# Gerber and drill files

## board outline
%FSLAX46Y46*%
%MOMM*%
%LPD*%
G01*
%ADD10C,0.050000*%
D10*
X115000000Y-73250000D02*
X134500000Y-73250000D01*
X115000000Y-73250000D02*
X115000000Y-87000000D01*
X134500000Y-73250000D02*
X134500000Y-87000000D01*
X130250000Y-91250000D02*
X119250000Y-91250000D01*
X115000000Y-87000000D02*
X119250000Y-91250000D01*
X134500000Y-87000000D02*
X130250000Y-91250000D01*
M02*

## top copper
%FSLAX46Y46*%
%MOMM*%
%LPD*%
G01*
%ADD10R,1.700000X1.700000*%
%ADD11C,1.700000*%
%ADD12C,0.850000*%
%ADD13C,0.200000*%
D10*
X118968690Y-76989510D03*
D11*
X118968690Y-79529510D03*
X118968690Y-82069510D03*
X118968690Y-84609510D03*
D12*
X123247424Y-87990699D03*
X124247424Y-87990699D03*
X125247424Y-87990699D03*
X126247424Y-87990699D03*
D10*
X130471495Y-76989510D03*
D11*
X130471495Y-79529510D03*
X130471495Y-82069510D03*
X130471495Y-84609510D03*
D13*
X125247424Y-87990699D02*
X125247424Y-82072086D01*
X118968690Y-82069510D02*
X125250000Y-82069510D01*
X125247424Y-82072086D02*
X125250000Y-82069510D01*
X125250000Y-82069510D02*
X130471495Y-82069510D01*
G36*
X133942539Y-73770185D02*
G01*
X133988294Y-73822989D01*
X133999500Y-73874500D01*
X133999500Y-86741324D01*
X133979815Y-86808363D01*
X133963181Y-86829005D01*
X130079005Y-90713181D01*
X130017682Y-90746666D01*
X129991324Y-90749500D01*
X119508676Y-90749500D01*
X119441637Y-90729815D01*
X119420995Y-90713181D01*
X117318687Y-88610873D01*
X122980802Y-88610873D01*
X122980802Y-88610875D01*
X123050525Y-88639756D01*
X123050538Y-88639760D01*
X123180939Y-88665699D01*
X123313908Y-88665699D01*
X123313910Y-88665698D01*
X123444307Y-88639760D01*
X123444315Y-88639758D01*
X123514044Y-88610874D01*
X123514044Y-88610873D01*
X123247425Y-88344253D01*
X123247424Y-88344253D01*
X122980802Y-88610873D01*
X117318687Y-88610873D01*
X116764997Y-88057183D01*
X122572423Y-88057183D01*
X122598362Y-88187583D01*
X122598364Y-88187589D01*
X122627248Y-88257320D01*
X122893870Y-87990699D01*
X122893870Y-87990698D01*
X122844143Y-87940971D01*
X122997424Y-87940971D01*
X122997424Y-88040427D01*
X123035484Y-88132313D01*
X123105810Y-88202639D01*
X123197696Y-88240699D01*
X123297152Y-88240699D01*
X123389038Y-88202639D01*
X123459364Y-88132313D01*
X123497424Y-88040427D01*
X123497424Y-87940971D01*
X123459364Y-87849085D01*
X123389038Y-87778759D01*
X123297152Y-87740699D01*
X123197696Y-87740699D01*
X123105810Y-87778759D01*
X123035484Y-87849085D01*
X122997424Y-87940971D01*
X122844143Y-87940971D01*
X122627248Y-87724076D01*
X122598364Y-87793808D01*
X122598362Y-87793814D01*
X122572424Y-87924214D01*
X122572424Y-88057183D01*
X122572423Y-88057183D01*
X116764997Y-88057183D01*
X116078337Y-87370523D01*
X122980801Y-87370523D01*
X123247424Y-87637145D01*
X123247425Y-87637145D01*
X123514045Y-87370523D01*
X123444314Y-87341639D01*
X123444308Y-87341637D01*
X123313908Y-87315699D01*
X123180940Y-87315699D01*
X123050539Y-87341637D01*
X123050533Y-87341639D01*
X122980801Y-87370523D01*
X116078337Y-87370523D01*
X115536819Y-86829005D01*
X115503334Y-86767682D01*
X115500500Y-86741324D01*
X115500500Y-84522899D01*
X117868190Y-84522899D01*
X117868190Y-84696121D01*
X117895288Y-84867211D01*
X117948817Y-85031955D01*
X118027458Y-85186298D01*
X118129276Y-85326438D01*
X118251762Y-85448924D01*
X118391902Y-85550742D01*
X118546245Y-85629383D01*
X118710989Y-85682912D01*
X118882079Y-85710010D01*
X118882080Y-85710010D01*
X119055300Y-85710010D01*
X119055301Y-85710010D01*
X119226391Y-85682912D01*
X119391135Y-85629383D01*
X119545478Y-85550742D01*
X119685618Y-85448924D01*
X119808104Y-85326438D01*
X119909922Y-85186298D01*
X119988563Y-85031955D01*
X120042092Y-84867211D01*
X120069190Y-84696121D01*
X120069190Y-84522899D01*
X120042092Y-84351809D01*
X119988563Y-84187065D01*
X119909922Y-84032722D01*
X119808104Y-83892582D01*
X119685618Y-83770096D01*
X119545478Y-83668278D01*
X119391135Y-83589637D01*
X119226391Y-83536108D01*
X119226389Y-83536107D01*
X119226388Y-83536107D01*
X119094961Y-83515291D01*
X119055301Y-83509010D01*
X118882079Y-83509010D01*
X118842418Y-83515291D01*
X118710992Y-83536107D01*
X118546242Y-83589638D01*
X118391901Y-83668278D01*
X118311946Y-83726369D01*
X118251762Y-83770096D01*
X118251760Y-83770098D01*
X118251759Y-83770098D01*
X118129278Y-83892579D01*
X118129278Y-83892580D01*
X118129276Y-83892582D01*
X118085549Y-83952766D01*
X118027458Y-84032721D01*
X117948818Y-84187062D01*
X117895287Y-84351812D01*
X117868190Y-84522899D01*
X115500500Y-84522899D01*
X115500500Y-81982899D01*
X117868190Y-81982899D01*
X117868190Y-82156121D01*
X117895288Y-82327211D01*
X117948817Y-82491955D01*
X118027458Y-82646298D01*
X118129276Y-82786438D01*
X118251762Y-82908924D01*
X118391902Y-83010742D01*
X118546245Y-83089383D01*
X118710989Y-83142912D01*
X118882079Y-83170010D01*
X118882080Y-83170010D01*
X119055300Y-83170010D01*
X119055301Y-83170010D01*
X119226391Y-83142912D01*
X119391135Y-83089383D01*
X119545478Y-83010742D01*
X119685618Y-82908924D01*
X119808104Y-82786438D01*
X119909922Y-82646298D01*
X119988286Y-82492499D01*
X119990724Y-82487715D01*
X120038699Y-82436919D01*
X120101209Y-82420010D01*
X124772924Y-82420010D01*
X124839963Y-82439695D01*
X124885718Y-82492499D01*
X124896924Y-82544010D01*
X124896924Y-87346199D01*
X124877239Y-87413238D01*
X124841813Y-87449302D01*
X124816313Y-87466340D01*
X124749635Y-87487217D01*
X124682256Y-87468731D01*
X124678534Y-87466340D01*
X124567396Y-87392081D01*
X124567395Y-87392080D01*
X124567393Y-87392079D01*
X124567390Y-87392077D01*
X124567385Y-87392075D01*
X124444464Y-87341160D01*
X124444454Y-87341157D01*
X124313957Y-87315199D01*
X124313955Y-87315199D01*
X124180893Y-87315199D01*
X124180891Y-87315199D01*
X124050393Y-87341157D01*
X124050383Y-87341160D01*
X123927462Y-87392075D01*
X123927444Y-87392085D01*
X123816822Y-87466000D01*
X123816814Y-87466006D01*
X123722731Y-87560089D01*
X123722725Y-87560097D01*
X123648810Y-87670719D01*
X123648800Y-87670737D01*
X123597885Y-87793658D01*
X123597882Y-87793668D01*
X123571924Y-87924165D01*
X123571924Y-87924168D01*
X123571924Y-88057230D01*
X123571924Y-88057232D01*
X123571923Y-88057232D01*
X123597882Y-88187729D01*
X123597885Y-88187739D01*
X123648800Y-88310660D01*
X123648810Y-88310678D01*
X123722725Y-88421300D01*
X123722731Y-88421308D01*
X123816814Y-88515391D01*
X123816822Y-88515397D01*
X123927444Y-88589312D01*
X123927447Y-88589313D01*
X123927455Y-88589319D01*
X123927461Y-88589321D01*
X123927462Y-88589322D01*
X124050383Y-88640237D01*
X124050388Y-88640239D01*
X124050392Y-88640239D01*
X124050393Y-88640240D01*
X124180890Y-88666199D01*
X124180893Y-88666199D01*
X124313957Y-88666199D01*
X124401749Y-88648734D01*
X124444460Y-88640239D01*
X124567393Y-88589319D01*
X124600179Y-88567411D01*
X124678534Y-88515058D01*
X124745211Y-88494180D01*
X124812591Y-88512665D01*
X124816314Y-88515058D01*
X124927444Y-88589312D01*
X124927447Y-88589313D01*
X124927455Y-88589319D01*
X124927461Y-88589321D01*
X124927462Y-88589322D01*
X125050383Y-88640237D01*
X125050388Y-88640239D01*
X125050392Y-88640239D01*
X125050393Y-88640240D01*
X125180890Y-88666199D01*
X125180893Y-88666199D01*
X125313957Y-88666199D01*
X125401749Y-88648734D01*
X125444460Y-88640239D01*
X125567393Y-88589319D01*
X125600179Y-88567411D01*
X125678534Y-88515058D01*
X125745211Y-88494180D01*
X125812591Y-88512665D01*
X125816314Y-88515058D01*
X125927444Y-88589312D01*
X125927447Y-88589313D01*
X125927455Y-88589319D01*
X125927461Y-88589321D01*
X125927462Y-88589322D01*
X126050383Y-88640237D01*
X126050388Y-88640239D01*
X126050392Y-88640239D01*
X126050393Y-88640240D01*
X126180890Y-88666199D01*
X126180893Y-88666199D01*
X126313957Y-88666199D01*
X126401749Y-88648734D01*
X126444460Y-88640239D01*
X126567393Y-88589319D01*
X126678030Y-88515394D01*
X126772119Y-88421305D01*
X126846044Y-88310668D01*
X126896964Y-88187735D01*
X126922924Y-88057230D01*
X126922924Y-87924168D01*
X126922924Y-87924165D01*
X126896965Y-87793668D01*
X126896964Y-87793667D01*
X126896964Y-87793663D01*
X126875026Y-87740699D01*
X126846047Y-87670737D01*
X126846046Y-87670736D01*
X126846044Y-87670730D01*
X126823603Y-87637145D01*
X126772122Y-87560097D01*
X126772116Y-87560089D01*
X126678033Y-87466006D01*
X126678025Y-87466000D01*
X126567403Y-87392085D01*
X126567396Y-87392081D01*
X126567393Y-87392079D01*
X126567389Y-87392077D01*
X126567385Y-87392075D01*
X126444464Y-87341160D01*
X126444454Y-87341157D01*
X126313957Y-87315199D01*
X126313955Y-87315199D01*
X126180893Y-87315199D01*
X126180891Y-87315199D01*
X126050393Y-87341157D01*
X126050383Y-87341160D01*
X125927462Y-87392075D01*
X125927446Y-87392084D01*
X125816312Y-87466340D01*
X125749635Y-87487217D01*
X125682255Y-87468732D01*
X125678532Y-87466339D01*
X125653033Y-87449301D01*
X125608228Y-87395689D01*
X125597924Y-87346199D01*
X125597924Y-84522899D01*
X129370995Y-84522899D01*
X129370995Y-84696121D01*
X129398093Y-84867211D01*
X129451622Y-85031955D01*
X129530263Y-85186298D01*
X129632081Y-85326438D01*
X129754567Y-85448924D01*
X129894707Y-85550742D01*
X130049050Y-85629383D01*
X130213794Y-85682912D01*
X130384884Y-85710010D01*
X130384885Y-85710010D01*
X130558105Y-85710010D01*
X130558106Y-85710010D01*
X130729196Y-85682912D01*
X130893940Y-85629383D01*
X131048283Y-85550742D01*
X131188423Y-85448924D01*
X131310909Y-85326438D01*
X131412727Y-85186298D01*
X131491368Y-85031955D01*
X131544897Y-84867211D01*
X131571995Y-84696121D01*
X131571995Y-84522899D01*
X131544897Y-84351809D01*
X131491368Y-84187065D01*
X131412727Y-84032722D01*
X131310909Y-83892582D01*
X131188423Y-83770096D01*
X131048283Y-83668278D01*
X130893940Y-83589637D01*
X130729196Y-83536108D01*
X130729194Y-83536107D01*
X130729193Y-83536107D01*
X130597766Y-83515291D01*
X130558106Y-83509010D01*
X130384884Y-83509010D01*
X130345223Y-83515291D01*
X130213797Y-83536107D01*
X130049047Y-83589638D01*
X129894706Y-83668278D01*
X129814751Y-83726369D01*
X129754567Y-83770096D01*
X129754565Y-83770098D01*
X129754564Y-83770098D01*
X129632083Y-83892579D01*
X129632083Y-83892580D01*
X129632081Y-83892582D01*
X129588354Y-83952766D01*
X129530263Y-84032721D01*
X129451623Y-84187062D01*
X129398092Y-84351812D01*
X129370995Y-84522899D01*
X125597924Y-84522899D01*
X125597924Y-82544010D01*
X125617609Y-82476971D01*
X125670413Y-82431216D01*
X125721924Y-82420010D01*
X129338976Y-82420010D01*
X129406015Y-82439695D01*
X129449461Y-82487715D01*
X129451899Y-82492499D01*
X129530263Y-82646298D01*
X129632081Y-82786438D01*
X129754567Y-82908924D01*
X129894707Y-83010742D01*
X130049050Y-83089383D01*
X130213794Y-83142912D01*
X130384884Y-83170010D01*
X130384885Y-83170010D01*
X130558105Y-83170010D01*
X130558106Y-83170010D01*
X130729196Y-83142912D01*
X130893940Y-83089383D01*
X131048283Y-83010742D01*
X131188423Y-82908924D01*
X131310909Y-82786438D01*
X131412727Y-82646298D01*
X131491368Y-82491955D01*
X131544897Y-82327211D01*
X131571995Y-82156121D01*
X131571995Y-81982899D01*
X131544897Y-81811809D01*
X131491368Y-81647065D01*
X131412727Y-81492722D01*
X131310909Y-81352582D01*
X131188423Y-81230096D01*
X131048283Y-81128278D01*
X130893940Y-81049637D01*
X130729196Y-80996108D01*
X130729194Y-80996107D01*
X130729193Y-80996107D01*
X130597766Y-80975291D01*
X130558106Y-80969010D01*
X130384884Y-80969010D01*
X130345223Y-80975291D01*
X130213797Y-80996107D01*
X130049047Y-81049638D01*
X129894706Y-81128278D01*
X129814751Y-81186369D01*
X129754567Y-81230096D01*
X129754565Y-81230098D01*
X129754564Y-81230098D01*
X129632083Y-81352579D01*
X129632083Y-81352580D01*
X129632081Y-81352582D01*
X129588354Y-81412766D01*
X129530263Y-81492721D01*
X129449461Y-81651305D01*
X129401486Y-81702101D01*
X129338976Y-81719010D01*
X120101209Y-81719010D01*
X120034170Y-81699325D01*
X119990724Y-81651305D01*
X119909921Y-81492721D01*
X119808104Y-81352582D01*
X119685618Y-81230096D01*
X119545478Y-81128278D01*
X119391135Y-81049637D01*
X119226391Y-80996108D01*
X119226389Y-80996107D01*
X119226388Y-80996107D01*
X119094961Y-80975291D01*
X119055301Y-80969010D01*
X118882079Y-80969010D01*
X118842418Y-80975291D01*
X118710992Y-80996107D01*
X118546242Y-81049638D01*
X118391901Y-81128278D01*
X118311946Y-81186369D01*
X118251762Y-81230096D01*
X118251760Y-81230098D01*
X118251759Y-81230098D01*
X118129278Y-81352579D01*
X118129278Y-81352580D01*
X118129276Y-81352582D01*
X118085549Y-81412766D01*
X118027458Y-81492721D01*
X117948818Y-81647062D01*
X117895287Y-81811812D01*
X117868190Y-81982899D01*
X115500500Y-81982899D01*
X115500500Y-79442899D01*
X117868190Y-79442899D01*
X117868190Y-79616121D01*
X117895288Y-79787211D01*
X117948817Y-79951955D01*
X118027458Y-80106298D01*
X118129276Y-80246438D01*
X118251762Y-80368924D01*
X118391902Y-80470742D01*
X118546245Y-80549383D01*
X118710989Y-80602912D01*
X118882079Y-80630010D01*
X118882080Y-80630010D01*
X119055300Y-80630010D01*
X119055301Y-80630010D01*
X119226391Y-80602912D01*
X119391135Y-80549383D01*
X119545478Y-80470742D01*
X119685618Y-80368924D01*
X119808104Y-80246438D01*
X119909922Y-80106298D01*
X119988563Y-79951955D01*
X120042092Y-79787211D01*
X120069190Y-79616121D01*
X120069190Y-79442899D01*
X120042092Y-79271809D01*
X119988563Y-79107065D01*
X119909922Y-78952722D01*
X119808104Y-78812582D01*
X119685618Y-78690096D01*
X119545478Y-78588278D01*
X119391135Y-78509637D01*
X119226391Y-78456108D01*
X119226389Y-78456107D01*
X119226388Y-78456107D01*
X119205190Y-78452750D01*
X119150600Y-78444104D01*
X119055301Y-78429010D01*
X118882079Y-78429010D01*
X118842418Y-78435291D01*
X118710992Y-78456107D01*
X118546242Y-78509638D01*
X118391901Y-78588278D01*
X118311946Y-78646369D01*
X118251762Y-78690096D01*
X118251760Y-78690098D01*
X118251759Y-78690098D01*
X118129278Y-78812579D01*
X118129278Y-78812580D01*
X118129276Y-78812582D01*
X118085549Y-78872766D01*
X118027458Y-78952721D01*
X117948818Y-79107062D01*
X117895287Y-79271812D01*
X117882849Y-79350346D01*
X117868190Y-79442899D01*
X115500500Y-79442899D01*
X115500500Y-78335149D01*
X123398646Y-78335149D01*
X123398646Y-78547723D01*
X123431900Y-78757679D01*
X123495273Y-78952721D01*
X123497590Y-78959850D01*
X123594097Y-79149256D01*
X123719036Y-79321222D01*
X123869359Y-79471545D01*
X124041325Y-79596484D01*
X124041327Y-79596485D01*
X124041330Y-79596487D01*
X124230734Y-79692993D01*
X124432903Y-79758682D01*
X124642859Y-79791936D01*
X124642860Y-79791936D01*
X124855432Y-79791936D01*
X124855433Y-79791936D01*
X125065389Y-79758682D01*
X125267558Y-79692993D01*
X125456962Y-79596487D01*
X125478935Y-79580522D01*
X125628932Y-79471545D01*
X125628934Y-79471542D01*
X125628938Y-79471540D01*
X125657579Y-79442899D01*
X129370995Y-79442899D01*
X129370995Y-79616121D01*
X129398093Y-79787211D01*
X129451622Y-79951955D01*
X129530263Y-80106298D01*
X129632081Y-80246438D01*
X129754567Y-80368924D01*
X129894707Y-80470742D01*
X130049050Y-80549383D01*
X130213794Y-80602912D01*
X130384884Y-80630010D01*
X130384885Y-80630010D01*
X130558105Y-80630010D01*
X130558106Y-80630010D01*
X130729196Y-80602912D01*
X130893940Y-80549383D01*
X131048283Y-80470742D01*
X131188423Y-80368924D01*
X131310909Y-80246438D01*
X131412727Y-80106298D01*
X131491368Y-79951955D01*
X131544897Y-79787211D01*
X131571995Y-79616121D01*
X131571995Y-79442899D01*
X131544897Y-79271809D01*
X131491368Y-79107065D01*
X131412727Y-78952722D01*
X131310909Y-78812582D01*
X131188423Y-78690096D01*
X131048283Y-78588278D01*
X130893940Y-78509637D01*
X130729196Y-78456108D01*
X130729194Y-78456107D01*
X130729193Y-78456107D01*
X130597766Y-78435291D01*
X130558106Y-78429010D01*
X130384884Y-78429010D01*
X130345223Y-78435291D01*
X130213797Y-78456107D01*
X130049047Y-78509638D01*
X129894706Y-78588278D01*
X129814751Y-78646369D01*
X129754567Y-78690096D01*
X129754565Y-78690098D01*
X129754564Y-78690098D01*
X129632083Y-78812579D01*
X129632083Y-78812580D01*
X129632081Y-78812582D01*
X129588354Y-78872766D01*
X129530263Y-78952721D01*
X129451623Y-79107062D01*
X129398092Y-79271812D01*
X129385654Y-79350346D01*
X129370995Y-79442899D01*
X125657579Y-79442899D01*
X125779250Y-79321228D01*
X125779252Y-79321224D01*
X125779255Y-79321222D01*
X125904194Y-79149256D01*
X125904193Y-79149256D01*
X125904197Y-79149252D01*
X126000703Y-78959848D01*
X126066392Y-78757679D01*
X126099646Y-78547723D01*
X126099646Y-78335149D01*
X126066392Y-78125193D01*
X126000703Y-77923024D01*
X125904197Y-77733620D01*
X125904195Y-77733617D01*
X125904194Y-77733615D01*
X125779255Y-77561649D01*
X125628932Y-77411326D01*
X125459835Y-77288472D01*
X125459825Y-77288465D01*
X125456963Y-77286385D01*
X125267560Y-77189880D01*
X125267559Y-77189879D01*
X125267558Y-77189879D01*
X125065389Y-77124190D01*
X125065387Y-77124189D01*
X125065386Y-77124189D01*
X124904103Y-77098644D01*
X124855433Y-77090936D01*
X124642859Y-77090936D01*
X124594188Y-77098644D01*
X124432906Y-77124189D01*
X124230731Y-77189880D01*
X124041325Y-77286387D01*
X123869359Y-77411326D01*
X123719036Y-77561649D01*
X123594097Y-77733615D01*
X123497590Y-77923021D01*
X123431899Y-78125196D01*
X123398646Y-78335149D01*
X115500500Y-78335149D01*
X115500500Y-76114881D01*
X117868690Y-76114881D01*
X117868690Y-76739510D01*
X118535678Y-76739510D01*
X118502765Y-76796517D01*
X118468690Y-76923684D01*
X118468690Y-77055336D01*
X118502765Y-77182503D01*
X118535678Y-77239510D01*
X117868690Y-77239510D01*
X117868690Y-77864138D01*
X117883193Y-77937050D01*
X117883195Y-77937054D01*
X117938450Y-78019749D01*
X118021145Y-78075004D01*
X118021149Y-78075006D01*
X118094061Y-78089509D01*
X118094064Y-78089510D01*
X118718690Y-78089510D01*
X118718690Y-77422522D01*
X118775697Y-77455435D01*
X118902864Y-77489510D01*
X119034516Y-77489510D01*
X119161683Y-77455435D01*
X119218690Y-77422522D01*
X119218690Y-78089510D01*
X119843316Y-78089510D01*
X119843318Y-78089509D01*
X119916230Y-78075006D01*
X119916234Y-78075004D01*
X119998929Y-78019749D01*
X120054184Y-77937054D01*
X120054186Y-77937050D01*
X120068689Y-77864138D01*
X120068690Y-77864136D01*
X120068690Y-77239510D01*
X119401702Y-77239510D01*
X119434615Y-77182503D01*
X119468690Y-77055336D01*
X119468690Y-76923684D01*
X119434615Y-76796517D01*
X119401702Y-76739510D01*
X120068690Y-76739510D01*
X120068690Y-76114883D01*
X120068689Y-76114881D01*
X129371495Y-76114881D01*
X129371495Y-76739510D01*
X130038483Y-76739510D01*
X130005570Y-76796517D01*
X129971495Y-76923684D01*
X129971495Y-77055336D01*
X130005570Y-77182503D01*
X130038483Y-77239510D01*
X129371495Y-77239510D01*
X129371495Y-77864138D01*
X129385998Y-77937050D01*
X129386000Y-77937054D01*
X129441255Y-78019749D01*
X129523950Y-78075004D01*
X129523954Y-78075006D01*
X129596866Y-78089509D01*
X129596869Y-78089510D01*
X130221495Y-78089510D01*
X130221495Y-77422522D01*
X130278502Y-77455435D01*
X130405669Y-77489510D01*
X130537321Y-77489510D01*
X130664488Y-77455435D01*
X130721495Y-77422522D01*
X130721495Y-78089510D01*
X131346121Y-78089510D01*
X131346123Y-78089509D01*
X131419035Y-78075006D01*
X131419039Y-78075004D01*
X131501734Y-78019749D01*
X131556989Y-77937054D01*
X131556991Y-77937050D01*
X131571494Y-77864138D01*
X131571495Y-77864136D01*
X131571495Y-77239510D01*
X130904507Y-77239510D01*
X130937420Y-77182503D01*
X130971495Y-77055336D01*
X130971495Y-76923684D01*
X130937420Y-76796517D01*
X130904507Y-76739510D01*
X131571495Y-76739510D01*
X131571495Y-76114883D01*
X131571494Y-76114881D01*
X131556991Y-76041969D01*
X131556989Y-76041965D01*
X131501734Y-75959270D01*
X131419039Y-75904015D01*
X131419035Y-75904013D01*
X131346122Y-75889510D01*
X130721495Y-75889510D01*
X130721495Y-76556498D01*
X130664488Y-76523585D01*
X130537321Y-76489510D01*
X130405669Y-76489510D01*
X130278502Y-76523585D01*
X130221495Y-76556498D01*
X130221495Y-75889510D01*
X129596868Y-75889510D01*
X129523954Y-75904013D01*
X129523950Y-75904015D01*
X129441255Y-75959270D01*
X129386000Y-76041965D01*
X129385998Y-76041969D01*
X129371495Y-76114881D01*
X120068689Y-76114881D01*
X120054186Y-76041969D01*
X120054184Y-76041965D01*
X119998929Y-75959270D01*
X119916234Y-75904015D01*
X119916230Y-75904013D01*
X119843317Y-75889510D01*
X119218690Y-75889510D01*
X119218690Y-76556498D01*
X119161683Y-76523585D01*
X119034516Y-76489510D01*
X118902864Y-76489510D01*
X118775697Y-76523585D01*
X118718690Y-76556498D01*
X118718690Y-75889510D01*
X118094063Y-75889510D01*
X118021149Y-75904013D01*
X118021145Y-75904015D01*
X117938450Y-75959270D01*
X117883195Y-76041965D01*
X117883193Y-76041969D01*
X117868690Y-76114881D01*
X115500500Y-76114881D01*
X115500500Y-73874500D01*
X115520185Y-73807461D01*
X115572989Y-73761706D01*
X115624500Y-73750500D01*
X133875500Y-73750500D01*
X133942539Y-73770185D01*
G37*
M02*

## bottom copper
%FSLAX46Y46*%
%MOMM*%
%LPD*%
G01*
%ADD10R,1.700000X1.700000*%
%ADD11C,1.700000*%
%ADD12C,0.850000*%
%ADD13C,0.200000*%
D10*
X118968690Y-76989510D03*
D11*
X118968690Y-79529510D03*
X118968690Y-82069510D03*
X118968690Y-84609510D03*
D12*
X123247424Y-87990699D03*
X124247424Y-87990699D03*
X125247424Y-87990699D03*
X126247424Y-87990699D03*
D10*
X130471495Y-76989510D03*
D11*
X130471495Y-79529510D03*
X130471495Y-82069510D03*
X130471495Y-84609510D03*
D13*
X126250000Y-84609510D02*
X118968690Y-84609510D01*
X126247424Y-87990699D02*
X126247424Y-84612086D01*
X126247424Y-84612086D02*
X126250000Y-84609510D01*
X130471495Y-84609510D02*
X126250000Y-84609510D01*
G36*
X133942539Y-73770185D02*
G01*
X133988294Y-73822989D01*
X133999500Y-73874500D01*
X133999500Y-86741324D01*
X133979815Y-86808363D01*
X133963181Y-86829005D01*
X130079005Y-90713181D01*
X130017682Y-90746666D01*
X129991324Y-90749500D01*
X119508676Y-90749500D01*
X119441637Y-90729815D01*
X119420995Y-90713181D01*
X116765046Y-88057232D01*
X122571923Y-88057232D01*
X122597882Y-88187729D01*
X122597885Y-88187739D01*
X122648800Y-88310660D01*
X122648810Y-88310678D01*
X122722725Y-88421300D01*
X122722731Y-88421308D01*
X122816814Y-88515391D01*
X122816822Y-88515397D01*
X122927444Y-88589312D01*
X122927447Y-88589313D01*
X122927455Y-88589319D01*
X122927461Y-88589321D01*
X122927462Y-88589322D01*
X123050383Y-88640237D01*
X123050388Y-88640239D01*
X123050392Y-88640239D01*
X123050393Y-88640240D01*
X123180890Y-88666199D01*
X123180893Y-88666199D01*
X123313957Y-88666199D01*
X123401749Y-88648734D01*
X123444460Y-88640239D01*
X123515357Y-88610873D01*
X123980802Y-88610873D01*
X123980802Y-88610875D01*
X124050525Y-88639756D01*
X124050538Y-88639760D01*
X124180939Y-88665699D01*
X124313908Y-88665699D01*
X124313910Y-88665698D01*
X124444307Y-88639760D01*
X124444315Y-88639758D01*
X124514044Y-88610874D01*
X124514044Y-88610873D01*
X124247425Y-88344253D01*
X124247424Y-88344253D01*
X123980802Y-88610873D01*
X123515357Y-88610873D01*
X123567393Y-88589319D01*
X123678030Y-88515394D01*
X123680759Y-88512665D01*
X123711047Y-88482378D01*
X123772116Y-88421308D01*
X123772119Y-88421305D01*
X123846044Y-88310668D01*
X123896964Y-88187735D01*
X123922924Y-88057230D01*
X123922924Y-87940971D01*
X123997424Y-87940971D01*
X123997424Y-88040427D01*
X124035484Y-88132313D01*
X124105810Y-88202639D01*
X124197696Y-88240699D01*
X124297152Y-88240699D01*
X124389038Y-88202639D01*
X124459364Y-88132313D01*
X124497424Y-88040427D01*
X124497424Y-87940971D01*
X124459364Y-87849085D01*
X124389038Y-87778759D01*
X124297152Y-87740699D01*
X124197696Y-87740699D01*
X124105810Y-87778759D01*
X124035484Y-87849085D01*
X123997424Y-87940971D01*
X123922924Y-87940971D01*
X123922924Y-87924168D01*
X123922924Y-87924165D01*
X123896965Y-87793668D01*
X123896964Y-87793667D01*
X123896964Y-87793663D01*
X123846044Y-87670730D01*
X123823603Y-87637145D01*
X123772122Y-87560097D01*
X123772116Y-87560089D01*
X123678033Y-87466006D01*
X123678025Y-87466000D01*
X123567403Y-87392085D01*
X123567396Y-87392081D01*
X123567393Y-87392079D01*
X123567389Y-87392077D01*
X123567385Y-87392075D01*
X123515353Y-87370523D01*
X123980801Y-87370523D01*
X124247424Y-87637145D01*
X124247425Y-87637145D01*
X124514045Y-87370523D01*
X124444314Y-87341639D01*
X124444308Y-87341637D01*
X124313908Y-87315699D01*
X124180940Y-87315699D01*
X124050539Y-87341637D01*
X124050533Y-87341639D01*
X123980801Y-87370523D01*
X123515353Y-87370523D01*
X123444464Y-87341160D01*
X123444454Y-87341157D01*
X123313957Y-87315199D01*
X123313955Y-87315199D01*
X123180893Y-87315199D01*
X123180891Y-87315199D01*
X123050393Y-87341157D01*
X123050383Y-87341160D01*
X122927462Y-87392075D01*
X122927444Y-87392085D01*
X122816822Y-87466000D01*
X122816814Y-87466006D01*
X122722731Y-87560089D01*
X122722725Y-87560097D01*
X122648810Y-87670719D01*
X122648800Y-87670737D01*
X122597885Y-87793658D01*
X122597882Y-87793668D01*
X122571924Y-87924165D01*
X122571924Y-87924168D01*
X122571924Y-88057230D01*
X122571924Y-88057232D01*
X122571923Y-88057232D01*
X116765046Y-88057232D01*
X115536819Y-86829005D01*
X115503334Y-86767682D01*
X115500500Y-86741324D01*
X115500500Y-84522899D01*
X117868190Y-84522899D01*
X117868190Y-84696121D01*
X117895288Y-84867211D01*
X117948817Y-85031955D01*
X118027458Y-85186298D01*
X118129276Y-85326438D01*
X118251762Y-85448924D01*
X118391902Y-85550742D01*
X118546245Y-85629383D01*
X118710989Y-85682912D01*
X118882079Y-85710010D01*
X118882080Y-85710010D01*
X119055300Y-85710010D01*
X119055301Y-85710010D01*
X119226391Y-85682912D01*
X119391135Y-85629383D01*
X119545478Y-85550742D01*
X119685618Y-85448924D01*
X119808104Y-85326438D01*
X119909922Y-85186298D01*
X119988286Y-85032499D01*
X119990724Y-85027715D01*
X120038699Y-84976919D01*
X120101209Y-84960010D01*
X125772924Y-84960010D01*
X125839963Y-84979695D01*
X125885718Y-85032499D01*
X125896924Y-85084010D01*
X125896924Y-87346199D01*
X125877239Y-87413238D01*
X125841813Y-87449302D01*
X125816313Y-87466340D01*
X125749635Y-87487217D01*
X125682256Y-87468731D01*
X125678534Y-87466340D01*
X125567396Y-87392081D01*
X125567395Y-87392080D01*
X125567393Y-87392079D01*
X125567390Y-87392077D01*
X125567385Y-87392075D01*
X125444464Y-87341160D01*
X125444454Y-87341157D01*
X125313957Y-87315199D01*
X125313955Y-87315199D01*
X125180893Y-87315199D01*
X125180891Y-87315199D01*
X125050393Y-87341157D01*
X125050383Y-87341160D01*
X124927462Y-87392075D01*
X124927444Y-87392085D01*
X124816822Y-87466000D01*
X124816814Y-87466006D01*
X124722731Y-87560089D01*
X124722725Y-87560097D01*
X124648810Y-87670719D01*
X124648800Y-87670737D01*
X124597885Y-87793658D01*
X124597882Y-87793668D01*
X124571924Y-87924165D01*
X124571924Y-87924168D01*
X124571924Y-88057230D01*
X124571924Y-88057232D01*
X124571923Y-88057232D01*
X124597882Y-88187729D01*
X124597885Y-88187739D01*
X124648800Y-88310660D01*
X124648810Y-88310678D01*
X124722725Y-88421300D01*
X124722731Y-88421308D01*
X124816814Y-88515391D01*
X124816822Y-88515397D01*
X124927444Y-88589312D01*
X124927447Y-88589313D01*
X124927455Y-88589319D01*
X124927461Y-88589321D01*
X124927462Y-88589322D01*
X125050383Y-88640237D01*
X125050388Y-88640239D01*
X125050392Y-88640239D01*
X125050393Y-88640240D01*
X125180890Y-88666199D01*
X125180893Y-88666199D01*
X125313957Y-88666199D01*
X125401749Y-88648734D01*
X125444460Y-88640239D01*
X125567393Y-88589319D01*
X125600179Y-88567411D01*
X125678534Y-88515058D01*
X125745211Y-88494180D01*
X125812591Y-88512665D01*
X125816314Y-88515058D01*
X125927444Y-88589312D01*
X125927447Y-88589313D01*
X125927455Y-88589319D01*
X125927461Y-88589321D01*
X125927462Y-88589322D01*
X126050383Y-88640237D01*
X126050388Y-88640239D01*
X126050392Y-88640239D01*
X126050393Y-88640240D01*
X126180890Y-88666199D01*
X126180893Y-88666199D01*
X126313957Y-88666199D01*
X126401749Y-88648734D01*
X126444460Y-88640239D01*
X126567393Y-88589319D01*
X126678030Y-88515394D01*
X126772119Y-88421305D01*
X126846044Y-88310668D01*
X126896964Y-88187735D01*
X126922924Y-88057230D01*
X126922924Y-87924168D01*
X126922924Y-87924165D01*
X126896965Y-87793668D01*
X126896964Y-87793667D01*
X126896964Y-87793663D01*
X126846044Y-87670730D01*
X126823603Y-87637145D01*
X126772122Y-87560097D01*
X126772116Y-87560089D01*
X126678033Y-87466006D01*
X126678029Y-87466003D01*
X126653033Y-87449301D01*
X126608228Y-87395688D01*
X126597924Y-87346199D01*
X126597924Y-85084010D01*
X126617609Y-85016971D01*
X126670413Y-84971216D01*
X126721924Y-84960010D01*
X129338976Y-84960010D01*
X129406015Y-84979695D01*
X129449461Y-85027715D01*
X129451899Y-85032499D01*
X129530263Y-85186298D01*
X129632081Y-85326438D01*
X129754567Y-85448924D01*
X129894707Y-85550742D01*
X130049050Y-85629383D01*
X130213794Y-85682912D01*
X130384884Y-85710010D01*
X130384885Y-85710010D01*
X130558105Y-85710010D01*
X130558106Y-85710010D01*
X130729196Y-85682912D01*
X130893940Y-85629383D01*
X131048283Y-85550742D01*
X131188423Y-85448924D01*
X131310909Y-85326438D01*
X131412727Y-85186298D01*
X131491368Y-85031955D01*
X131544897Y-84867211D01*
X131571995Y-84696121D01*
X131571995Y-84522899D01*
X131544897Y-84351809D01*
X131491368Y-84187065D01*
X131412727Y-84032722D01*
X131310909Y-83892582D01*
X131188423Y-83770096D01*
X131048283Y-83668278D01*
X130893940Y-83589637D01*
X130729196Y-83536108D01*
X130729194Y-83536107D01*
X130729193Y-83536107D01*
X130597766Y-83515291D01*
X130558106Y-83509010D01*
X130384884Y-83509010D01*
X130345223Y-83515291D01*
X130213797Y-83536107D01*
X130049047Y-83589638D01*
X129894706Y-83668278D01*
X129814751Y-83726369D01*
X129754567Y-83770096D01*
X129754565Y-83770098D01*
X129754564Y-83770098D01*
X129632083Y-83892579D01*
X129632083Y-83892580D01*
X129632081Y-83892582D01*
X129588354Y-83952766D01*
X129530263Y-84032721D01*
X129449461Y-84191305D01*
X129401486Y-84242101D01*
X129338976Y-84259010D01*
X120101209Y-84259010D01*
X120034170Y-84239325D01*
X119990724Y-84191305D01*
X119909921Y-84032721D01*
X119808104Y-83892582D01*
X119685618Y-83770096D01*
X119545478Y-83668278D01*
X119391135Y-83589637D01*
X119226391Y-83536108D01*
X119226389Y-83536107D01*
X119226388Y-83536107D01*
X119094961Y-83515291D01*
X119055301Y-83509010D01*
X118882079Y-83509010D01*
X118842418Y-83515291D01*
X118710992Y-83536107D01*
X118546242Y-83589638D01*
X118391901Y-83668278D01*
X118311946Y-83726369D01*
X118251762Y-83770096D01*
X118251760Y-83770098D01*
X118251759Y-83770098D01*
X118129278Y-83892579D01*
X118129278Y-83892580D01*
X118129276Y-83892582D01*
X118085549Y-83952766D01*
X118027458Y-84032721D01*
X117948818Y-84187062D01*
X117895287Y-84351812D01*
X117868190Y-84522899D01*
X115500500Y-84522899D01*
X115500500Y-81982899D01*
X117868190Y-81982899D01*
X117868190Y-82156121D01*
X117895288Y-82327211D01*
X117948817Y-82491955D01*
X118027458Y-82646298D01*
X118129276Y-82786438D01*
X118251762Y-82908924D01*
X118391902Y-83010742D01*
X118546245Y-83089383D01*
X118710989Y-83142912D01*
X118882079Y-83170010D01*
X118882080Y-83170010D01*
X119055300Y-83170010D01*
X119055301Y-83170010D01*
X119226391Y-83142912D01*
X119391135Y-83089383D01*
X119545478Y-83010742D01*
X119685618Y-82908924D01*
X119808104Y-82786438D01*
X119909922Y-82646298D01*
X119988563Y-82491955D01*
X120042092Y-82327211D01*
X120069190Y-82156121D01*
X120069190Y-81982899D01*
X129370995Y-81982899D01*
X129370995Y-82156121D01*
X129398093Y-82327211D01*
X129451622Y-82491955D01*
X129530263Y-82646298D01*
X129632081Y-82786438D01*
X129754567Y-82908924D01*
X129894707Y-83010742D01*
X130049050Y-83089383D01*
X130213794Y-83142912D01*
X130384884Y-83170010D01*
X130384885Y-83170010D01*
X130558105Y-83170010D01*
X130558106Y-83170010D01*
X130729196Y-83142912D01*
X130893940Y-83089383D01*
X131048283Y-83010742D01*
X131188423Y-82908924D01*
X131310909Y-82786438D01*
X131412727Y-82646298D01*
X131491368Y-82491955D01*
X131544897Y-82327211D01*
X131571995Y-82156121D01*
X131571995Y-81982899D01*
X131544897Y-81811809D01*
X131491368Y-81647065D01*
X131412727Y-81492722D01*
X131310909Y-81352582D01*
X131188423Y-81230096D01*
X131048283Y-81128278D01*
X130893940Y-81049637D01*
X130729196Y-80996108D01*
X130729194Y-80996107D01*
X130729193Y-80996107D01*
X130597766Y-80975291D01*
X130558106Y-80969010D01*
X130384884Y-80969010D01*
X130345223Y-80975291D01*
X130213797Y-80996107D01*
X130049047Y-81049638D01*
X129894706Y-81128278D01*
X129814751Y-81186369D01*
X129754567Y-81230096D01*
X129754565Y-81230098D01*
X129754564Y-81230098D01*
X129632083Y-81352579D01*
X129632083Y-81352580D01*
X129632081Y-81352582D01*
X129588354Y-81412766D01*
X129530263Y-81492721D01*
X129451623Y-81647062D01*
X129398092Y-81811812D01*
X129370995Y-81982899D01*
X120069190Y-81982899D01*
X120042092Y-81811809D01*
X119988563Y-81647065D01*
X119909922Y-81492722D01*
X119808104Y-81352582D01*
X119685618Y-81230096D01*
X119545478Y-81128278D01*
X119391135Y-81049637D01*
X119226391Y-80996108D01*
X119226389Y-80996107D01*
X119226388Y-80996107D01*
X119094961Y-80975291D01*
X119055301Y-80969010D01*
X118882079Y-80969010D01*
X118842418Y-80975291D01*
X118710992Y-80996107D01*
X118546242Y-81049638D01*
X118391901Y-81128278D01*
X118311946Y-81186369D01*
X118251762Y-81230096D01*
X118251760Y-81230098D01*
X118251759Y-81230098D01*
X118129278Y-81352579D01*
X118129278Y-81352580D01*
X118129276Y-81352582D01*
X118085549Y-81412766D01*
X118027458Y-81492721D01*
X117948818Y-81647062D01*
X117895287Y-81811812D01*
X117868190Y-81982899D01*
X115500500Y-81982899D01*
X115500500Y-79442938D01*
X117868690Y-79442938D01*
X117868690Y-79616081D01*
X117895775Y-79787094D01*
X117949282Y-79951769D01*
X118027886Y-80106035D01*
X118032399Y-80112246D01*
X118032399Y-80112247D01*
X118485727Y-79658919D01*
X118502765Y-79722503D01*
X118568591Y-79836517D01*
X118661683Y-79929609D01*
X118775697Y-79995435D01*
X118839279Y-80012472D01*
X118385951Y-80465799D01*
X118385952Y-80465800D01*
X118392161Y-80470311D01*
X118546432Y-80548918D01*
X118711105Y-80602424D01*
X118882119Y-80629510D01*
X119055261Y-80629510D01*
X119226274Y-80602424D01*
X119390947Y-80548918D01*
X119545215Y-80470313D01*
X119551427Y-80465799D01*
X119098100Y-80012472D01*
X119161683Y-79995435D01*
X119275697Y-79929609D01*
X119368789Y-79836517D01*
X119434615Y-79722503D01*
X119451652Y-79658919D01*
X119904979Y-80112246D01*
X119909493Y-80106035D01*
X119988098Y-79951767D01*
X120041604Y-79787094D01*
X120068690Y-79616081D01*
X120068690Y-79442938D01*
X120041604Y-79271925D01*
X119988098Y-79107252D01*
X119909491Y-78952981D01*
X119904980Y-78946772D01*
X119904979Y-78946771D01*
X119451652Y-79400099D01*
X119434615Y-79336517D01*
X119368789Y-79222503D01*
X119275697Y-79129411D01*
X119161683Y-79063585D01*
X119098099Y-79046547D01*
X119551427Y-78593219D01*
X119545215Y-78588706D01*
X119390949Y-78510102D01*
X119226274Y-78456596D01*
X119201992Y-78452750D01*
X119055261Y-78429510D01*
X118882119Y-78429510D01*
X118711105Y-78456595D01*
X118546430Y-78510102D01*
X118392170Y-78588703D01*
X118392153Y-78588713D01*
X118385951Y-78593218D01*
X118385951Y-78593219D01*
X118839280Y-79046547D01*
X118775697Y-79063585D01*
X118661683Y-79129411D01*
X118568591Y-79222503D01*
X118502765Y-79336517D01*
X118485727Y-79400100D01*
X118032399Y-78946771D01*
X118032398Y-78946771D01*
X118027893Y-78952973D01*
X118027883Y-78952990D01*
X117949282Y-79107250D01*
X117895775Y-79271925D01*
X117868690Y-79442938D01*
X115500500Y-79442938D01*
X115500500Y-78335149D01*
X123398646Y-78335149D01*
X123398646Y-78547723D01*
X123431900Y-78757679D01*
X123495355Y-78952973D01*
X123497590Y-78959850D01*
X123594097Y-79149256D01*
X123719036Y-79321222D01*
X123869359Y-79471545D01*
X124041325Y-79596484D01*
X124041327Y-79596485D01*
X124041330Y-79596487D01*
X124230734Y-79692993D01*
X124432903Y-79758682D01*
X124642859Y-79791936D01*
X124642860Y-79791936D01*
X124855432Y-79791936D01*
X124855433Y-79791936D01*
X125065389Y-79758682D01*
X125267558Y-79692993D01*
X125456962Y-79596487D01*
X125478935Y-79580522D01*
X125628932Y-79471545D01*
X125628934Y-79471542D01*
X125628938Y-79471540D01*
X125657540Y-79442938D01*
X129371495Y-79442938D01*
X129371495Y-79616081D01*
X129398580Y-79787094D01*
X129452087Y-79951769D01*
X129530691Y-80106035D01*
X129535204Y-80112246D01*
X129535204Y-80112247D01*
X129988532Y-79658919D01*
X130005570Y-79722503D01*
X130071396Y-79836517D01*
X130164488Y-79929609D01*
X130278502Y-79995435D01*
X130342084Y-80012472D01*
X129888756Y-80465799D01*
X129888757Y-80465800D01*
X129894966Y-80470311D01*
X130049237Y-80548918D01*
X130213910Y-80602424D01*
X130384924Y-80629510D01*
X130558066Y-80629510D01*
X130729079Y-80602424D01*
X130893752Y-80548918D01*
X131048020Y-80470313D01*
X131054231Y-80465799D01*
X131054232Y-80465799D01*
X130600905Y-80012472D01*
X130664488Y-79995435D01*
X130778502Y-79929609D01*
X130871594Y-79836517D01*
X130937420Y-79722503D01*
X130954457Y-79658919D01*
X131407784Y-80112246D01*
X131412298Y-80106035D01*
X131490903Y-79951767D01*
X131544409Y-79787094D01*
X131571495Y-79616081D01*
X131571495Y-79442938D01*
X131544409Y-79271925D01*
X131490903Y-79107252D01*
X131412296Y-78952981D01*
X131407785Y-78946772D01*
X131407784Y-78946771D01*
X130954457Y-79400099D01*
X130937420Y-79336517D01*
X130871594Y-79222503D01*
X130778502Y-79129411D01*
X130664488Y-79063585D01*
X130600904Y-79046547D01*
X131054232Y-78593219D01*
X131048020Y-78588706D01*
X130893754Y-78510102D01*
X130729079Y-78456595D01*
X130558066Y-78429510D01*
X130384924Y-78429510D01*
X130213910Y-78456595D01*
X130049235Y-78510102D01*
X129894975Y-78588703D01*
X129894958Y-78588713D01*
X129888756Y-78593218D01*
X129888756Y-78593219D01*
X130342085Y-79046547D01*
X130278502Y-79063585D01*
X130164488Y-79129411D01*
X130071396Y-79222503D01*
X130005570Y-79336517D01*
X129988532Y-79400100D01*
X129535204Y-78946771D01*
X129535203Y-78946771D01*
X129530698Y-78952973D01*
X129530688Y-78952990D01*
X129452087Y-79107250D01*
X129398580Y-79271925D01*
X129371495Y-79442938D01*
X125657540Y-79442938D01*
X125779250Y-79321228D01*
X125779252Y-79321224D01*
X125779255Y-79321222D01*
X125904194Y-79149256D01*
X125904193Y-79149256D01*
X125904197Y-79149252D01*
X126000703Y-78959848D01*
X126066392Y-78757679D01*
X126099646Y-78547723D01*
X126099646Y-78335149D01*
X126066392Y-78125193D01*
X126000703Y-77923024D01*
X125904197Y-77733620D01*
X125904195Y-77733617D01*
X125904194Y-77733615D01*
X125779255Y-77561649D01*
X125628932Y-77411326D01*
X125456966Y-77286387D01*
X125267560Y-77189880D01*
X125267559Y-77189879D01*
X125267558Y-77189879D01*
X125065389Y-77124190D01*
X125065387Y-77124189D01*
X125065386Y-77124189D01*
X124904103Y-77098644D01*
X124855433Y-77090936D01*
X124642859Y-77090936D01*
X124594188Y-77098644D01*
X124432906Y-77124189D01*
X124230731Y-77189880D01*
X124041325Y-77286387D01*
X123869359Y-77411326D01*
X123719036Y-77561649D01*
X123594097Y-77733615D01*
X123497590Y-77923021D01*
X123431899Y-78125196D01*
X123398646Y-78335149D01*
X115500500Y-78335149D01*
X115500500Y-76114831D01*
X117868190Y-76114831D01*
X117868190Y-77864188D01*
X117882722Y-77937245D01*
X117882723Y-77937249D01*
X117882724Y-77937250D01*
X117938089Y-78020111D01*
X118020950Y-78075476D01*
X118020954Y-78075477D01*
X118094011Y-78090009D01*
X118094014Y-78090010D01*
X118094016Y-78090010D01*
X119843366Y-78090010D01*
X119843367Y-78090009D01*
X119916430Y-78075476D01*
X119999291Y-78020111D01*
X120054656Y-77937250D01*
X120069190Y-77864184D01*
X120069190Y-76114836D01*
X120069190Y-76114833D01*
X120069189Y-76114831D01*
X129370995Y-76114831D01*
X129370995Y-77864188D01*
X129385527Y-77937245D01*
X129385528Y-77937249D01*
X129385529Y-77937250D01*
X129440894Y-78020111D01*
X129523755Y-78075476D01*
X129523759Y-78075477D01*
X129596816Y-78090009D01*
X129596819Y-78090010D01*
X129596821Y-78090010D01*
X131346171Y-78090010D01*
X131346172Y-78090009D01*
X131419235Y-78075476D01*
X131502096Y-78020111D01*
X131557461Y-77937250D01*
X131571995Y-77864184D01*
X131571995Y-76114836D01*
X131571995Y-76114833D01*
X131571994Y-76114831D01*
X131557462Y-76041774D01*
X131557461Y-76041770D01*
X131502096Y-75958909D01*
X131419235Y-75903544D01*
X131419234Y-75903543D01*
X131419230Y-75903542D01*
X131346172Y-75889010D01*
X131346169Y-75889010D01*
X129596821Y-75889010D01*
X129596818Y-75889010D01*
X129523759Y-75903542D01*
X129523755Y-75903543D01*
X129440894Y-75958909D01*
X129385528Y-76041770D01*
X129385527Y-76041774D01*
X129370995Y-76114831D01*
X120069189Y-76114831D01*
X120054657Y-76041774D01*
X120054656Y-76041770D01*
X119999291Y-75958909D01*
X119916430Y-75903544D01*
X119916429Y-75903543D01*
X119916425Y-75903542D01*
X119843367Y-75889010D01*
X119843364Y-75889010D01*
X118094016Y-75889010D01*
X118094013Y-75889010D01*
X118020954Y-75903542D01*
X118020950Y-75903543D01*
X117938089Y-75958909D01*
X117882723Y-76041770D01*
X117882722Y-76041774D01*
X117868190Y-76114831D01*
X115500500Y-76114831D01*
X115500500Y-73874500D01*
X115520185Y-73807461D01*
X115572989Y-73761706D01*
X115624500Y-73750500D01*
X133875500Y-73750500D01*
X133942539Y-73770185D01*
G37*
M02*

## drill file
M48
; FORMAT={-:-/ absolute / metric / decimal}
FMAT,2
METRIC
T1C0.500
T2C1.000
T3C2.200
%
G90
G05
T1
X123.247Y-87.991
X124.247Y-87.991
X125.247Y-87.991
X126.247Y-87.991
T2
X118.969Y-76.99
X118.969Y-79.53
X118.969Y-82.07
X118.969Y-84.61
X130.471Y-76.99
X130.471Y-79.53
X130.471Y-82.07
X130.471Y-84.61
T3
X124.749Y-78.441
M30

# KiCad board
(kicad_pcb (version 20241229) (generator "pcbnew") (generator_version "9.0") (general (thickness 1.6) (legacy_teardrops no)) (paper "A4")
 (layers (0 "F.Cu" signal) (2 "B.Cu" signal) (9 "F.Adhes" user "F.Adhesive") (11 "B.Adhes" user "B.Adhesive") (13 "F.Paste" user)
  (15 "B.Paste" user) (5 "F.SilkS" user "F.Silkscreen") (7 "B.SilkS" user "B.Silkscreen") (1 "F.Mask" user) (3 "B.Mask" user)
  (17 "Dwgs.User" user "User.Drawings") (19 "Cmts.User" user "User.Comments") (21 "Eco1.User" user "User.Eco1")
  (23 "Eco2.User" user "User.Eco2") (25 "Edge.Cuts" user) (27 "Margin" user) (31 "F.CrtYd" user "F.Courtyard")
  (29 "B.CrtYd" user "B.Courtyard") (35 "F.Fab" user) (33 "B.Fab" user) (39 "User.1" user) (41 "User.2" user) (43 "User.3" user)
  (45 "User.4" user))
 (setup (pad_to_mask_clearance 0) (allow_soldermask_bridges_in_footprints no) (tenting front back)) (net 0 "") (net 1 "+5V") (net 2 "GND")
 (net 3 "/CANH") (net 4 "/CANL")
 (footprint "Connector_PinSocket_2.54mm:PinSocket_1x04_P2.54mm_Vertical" (layer "F.Cu") (at 118.96869 76.98951)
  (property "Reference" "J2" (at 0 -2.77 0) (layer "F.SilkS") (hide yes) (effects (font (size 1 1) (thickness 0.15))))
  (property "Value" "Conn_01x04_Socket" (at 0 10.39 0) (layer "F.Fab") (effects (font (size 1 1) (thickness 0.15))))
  (pad "1" thru_hole rect (at 0 0) (size 1.7 1.7) (drill 1) (layers "*.Cu" "*.Mask") (remove_unused_layers no) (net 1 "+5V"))
  (pad "2" thru_hole circle (at 0 2.54) (size 1.7 1.7) (drill 1) (layers "*.Cu" "*.Mask") (remove_unused_layers no) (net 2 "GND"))
  (pad "3" thru_hole circle (at 0 5.08) (size 1.7 1.7) (drill 1) (layers "*.Cu" "*.Mask") (remove_unused_layers no) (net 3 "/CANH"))
  (pad "4" thru_hole circle (at 0 7.62) (size 1.7 1.7) (drill 1) (layers "*.Cu" "*.Mask") (remove_unused_layers no) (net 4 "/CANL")))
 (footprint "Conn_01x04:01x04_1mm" (layer "F.Cu") (at 122.747424 88.490699 90)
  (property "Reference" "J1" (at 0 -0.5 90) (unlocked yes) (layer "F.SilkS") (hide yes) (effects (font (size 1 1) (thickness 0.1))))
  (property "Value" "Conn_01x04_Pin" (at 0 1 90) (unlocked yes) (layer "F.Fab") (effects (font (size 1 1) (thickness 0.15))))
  (pad "1" thru_hole circle (at 0.5 0.5 90) (size 0.85 0.85) (drill 0.5) (layers "*.Cu" "*.Mask") (remove_unused_layers no) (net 1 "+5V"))
  (pad "2" thru_hole circle (at 0.5 1.5 90) (size 0.85 0.85) (drill 0.5) (layers "*.Cu" "*.Mask") (remove_unused_layers no) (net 2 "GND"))
  (pad "3" thru_hole circle (at 0.5 2.5 90) (size 0.85 0.85) (drill 0.5) (layers "*.Cu" "*.Mask") (remove_unused_layers no) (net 3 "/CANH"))
  (pad "4" thru_hole circle (at 0.5 3.5 90) (size 0.85 0.85) (drill 0.5) (layers "*.Cu" "*.Mask") (remove_unused_layers no) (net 4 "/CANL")))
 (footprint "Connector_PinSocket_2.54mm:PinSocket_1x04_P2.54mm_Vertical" (layer "F.Cu") (at 130.471495 76.98951)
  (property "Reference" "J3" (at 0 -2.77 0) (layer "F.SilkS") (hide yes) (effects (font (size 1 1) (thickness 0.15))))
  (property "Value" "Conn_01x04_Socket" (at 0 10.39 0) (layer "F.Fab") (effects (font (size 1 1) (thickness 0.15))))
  (pad "1" thru_hole rect (at 0 0) (size 1.7 1.7) (drill 1) (layers "*.Cu" "*.Mask") (remove_unused_layers no) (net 1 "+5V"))
  (pad "2" thru_hole circle (at 0 2.54) (size 1.7 1.7) (drill 1) (layers "*.Cu" "*.Mask") (remove_unused_layers no) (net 2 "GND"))
  (pad "3" thru_hole circle (at 0 5.08) (size 1.7 1.7) (drill 1) (layers "*.Cu" "*.Mask") (remove_unused_layers no) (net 3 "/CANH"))
  (pad "4" thru_hole circle (at 0 7.62) (size 1.7 1.7) (drill 1) (layers "*.Cu" "*.Mask") (remove_unused_layers no) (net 4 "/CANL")))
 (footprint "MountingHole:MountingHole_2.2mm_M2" (layer "F.Cu") (at 124.749146 78.441436)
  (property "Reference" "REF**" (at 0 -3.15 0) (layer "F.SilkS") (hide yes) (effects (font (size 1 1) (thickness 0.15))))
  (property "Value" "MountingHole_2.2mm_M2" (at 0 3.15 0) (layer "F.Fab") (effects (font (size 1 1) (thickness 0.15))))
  (pad "" np_thru_hole circle (at 0 0) (size 2.2 2.2) (drill 2.2) (layers "*.Cu" "*.Mask")))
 (gr_line (start 115 73.25) (end 134.5 73.25) (stroke (width 0.05) (type solid)) (layer "Edge.Cuts"))
 (gr_line (start 115 73.25) (end 115 87) (stroke (width 0.05) (type default)) (layer "Edge.Cuts"))
 (gr_line (start 134.5 73.25) (end 134.5 87) (stroke (width 0.05) (type default)) (layer "Edge.Cuts"))
 (gr_line (start 130.25 91.25) (end 119.25 91.25) (stroke (width 0.05) (type default)) (layer "Edge.Cuts"))
 (gr_line (start 115 87) (end 119.25 91.25) (stroke (width 0.05) (type default)) (layer "Edge.Cuts"))
 (gr_line (start 134.5 87) (end 130.25 91.25) (stroke (width 0.05) (type default)) (layer "Edge.Cuts"))
 (segment (start 126.25 84.60951) (end 118.96869 84.60951) (width 0.2) (layer "B.Cu") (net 4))
 (segment (start 126.247424 87.990699) (end 126.247424 84.612086) (width 0.2) (layer "B.Cu") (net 4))
 (segment (start 126.247424 84.612086) (end 126.25 84.60951) (width 0.2) (layer "B.Cu") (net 4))
 (segment (start 130.471495 84.60951) (end 126.25 84.60951) (width 0.2) (layer "B.Cu") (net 4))
 (segment (start 125.247424 87.990699) (end 125.247424 82.072086) (width 0.2) (layer "F.Cu") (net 3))
 (segment (start 118.96869 82.06951) (end 125.25 82.06951) (width 0.2) (layer "F.Cu") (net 3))
 (segment (start 125.247424 82.072086) (end 125.25 82.06951) (width 0.2) (layer "F.Cu") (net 3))
 (segment (start 125.25 82.06951) (end 130.471495 82.06951) (width 0.2) (layer "F.Cu") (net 3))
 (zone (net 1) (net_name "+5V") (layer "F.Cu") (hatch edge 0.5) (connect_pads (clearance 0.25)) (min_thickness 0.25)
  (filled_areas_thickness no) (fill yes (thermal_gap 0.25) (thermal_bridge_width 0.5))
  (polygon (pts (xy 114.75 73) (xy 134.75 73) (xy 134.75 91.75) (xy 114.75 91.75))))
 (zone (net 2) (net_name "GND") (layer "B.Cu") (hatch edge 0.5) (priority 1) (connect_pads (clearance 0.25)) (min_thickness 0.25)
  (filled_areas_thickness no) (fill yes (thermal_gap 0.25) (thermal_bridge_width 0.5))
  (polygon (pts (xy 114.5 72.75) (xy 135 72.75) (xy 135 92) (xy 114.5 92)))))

